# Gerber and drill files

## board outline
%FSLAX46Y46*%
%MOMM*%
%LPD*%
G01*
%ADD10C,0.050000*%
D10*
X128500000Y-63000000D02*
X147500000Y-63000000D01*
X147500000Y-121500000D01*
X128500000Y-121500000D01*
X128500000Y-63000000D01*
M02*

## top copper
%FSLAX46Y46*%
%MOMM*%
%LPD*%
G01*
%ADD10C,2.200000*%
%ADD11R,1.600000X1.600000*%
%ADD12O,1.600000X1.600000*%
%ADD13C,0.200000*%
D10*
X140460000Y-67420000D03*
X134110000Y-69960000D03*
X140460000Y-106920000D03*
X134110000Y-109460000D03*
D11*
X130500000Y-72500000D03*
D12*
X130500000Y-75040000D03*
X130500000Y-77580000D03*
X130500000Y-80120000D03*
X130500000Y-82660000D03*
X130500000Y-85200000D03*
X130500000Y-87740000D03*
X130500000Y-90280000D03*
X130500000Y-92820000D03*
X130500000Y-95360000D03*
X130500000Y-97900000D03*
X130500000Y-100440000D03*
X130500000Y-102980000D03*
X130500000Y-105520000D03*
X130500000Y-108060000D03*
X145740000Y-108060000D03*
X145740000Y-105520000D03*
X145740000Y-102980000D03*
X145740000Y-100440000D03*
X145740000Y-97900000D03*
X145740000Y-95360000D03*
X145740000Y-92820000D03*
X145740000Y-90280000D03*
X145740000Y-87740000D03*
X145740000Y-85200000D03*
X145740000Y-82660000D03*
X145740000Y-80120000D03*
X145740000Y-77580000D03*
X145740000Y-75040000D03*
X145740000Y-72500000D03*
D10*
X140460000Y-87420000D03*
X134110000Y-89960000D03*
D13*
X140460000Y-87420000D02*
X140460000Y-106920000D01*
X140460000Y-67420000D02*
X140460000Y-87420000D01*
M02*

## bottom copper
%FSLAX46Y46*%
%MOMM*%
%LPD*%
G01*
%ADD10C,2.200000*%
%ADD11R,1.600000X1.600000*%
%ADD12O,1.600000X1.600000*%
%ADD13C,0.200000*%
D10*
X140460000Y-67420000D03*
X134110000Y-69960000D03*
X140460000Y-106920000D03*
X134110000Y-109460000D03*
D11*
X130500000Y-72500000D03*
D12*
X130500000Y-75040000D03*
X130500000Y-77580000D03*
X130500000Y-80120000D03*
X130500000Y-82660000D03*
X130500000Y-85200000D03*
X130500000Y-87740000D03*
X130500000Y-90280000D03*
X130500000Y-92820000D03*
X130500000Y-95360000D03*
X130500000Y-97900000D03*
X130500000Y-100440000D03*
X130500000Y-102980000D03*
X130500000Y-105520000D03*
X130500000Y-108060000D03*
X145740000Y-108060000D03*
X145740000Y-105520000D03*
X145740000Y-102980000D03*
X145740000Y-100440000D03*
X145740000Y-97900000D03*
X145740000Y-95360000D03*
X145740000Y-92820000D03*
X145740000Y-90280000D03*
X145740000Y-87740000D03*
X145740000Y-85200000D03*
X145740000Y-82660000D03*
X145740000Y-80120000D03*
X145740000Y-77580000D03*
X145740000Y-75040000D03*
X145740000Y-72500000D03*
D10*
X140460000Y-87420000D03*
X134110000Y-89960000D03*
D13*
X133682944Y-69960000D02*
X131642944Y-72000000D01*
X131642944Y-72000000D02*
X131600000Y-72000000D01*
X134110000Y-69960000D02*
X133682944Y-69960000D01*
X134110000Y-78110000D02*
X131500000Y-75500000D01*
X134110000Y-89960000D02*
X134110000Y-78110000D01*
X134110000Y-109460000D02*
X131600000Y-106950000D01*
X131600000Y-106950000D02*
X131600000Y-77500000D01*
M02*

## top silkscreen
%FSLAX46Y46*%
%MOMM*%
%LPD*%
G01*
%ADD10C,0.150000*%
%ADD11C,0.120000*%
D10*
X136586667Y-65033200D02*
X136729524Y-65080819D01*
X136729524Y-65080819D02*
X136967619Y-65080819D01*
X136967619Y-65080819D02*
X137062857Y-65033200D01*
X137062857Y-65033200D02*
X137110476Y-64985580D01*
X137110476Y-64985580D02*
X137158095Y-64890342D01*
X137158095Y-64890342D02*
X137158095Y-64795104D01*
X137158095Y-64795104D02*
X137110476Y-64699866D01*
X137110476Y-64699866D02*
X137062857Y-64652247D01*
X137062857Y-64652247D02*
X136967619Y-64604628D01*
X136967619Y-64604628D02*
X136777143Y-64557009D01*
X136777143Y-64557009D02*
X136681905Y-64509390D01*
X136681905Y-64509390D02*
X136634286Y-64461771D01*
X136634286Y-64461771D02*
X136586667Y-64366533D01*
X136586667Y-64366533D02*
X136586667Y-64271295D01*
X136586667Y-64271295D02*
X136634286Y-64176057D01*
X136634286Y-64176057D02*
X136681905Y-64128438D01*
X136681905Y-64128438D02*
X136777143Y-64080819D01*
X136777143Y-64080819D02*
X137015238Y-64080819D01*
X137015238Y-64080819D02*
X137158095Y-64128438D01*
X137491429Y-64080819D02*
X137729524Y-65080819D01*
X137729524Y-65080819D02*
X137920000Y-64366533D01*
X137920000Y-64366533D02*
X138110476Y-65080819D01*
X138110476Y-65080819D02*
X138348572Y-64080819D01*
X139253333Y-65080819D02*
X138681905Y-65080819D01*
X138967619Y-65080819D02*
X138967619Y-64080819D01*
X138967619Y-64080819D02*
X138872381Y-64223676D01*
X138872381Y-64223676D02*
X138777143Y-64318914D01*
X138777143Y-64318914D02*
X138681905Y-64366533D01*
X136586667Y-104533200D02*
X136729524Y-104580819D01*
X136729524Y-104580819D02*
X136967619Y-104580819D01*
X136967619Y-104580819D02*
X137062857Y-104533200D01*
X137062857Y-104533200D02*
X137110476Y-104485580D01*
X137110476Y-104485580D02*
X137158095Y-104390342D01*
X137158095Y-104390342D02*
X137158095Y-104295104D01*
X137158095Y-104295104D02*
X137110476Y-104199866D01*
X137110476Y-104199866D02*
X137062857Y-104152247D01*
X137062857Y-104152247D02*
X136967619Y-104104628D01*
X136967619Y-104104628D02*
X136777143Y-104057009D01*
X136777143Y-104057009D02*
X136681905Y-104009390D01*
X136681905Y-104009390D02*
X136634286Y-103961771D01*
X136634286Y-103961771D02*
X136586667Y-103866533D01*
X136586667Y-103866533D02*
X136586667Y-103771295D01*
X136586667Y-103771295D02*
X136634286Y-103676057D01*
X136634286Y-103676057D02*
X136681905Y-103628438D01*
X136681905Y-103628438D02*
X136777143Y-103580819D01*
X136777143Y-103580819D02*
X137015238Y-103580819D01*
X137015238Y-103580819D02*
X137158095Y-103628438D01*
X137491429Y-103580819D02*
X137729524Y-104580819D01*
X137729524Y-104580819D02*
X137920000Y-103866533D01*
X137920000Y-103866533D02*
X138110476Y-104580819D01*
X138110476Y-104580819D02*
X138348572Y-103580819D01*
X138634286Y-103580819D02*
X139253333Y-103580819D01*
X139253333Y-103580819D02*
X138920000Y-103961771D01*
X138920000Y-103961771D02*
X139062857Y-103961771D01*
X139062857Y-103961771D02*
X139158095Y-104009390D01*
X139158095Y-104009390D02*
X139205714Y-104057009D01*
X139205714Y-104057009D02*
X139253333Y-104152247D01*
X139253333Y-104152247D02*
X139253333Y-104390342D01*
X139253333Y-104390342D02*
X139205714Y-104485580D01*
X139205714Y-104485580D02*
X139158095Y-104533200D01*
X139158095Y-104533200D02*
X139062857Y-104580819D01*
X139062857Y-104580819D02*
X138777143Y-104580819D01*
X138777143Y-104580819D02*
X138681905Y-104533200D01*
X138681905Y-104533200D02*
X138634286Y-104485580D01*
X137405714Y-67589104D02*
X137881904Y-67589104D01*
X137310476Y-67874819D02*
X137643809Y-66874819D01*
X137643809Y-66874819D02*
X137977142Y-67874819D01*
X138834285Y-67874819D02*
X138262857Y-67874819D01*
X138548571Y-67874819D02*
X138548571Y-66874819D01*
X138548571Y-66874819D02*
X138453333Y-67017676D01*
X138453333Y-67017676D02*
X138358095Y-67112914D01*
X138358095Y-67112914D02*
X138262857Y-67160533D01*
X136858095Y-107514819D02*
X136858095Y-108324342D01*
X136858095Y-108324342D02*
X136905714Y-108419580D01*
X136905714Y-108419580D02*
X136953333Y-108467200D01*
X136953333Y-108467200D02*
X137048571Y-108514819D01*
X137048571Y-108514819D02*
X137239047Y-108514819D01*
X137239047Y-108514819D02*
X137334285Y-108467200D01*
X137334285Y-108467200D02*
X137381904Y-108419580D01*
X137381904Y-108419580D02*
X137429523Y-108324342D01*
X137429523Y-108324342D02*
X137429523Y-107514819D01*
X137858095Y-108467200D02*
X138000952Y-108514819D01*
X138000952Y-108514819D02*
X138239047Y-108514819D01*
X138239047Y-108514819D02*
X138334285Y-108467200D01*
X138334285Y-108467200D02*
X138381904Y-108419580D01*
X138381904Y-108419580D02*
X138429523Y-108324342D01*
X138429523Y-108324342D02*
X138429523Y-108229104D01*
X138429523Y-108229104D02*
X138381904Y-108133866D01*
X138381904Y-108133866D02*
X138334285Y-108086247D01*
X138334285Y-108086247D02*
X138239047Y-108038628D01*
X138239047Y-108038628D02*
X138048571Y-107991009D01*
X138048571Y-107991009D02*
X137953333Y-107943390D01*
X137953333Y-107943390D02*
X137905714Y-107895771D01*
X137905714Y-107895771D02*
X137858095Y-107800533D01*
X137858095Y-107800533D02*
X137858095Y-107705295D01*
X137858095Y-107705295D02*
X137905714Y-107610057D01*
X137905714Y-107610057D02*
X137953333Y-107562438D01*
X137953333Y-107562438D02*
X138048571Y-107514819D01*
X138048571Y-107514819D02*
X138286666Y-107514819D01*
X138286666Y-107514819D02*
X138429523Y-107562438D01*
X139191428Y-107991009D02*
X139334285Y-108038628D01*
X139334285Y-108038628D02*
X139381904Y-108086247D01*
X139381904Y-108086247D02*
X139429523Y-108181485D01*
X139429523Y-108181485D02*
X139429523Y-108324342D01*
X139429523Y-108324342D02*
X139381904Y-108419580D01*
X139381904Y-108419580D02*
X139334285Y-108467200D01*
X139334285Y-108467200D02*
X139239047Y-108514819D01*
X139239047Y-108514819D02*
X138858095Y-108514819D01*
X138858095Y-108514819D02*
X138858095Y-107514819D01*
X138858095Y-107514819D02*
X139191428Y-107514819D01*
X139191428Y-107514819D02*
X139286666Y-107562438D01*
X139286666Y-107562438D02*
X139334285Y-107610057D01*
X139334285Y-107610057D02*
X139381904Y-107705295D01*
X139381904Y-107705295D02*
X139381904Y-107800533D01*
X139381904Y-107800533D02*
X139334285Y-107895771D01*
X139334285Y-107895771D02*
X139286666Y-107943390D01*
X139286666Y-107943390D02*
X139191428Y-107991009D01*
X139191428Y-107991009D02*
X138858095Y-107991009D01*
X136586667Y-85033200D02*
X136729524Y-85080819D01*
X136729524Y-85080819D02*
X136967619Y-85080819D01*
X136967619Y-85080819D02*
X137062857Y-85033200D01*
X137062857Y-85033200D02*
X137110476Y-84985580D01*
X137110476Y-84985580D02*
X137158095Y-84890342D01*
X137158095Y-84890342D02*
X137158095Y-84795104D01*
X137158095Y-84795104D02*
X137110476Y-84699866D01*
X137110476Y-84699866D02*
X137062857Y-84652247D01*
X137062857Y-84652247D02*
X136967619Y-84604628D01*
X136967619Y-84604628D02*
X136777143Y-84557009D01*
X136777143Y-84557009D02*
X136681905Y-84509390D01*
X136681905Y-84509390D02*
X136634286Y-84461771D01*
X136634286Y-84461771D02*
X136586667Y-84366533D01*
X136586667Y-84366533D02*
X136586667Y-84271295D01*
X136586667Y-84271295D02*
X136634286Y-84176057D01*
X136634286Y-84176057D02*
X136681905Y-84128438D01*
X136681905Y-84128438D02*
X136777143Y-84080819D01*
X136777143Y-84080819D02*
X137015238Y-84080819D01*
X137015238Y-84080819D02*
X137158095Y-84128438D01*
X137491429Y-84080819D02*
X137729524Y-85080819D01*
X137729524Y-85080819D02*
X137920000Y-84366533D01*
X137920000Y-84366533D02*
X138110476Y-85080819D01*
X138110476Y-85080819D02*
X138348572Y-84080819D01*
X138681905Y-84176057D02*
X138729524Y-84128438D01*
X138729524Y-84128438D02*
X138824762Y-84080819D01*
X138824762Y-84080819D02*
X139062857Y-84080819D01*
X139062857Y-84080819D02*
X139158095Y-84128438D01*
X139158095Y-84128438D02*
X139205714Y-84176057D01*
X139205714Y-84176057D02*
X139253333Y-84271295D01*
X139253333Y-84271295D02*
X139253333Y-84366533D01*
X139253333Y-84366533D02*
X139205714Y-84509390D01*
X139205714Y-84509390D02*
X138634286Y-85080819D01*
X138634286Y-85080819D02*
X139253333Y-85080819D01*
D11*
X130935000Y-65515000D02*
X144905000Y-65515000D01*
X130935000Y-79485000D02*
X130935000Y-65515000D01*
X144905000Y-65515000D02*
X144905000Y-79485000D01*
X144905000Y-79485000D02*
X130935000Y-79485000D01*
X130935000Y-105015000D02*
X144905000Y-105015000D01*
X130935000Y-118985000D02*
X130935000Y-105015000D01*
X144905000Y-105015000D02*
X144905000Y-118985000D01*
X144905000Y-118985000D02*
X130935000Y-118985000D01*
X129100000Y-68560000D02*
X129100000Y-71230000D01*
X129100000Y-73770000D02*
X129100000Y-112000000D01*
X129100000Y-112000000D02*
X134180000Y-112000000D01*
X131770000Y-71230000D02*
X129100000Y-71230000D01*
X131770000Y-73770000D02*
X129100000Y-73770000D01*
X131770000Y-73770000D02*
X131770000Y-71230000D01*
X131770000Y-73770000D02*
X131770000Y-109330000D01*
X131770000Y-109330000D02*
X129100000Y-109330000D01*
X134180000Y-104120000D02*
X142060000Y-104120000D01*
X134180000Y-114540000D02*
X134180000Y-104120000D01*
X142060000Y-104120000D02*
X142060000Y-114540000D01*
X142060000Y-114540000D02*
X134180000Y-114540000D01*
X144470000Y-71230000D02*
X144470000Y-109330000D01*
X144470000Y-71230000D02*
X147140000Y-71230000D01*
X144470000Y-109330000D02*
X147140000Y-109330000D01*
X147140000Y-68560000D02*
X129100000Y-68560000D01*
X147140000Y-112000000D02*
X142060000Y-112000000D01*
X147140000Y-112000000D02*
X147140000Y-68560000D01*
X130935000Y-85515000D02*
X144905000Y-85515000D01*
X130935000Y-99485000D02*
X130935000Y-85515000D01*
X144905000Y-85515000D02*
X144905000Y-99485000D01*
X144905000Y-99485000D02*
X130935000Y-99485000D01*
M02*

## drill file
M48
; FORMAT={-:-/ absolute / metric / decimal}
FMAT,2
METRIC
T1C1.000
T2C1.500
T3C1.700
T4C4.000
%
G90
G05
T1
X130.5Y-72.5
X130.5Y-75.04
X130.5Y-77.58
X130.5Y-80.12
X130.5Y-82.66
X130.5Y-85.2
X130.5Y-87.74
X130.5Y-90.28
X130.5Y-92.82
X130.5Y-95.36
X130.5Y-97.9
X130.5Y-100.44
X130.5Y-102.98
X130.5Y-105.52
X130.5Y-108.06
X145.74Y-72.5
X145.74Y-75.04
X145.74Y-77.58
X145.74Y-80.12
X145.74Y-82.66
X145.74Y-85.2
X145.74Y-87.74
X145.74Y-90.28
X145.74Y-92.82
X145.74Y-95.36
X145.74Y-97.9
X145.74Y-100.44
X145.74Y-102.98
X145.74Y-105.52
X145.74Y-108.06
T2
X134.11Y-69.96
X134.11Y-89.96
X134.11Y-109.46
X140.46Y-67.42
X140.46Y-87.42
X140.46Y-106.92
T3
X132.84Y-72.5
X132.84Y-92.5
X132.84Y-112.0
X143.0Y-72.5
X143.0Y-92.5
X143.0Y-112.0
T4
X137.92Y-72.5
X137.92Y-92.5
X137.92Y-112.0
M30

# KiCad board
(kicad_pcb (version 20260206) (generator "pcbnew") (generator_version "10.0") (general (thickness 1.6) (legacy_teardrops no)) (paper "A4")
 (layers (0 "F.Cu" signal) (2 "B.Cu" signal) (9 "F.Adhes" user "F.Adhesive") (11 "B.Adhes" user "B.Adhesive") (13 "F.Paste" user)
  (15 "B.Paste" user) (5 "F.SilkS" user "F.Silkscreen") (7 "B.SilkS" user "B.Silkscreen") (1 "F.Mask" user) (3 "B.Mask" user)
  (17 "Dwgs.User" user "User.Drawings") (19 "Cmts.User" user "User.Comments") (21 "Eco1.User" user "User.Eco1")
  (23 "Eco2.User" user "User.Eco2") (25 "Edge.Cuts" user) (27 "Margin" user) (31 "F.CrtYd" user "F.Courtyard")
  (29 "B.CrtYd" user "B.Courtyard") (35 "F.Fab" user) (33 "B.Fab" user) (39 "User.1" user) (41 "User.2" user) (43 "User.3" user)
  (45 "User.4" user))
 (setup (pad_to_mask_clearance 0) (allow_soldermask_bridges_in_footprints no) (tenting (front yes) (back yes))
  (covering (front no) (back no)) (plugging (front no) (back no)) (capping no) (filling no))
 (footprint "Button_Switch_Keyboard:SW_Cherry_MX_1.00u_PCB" (layer "F.Cu") (at 140.46 67.42)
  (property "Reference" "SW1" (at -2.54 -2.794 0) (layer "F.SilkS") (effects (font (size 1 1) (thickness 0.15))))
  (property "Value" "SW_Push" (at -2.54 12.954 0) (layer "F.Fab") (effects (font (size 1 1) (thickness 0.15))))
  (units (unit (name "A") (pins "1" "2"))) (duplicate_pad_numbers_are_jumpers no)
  (fp_line (start -9.525 -1.905) (end 4.445 -1.905) (stroke (width 0.12) (type solid)) (layer "F.SilkS"))
  (fp_line (start -9.525 12.065) (end -9.525 -1.905) (stroke (width 0.12) (type solid)) (layer "F.SilkS"))
  (fp_line (start 4.445 -1.905) (end 4.445 12.065) (stroke (width 0.12) (type solid)) (layer "F.SilkS"))
  (fp_line (start 4.445 12.065) (end -9.525 12.065) (stroke (width 0.12) (type solid)) (layer "F.SilkS"))
  (pad "" np_thru_hole circle (at -7.62 5.08) (size 1.7 1.7) (drill 1.7) (layers "*.Cu" "*.Mask"))
  (pad "" np_thru_hole circle (at -2.54 5.08) (size 4 4) (drill 4) (layers "*.Cu" "*.Mask"))
  (pad "" np_thru_hole circle (at 2.54 5.08) (size 1.7 1.7) (drill 1.7) (layers "*.Cu" "*.Mask"))
  (pad "1" thru_hole circle (at 0 0) (size 2.2 2.2) (drill 1.5) (layers "*.Cu" "*.Mask") (remove_unused_layers no) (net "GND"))
  (pad "2" thru_hole circle (at -6.35 2.54) (size 2.2 2.2) (drill 1.5) (layers "*.Cu" "*.Mask") (remove_unused_layers no)
   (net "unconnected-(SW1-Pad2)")))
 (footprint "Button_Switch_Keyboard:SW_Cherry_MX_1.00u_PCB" (layer "F.Cu") (at 140.46 106.92)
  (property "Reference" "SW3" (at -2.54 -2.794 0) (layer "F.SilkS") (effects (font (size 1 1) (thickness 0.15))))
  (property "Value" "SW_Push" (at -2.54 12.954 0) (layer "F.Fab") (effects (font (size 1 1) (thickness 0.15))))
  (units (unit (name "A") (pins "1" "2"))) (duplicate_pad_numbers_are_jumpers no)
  (fp_line (start -9.525 -1.905) (end 4.445 -1.905) (stroke (width 0.12) (type solid)) (layer "F.SilkS"))
  (fp_line (start -9.525 12.065) (end -9.525 -1.905) (stroke (width 0.12) (type solid)) (layer "F.SilkS"))
  (fp_line (start 4.445 -1.905) (end 4.445 12.065) (stroke (width 0.12) (type solid)) (layer "F.SilkS"))
  (fp_line (start 4.445 12.065) (end -9.525 12.065) (stroke (width 0.12) (type solid)) (layer "F.SilkS"))
  (pad "" np_thru_hole circle (at -7.62 5.08) (size 1.7 1.7) (drill 1.7) (layers "*.Cu" "*.Mask"))
  (pad "" np_thru_hole circle (at -2.54 5.08) (size 4 4) (drill 4) (layers "*.Cu" "*.Mask"))
  (pad "" np_thru_hole circle (at 2.54 5.08) (size 1.7 1.7) (drill 1.7) (layers "*.Cu" "*.Mask"))
  (pad "1" thru_hole circle (at 0 0) (size 2.2 2.2) (drill 1.5) (layers "*.Cu" "*.Mask") (remove_unused_layers no) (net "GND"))
  (pad "2" thru_hole circle (at -6.35 2.54) (size 2.2 2.2) (drill 1.5) (layers "*.Cu" "*.Mask") (remove_unused_layers no)
   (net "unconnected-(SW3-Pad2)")))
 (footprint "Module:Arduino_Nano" (layer "F.Cu") (at 130.5 72.5)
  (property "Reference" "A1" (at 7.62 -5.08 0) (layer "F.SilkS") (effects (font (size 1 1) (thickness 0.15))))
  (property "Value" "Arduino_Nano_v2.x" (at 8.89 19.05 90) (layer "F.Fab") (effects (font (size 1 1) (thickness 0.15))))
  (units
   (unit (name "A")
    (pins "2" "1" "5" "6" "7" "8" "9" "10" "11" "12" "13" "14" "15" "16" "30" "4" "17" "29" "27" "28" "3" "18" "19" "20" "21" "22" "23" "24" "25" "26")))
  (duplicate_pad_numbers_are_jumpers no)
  (fp_line (start -1.4 -3.94) (end -1.4 -1.27) (stroke (width 0.12) (type solid)) (layer "F.SilkS"))
  (fp_line (start -1.4 1.27) (end -1.4 39.5) (stroke (width 0.12) (type solid)) (layer "F.SilkS"))
  (fp_line (start -1.4 39.5) (end 3.68 39.5) (stroke (width 0.12) (type solid)) (layer "F.SilkS"))
  (fp_line (start 1.27 -1.27) (end -1.4 -1.27) (stroke (width 0.12) (type solid)) (layer "F.SilkS"))
  (fp_line (start 1.27 1.27) (end -1.4 1.27) (stroke (width 0.12) (type solid)) (layer "F.SilkS"))
  (fp_line (start 1.27 1.27) (end 1.27 -1.27) (stroke (width 0.12) (type solid)) (layer "F.SilkS"))
  (fp_line (start 1.27 1.27) (end 1.27 36.83) (stroke (width 0.12) (type solid)) (layer "F.SilkS"))
  (fp_line (start 1.27 36.83) (end -1.4 36.83) (stroke (width 0.12) (type solid)) (layer "F.SilkS"))
  (fp_line (start 3.68 31.62) (end 11.56 31.62) (stroke (width 0.12) (type solid)) (layer "F.SilkS"))
  (fp_line (start 3.68 42.04) (end 3.68 31.62) (stroke (width 0.12) (type solid)) (layer "F.SilkS"))
  (fp_line (start 11.56 31.62) (end 11.56 42.04) (stroke (width 0.12) (type solid)) (layer "F.SilkS"))
  (fp_line (start 11.56 42.04) (end 3.68 42.04) (stroke (width 0.12) (type solid)) (layer "F.SilkS"))
  (fp_line (start 13.97 -1.27) (end 13.97 36.83) (stroke (width 0.12) (type solid)) (layer "F.SilkS"))
  (fp_line (start 13.97 -1.27) (end 16.64 -1.27) (stroke (width 0.12) (type solid)) (layer "F.SilkS"))
  (fp_line (start 13.97 36.83) (end 16.64 36.83) (stroke (width 0.12) (type solid)) (layer "F.SilkS"))
  (fp_line (start 16.64 -3.94) (end -1.4 -3.94) (stroke (width 0.12) (type solid)) (layer "F.SilkS"))
  (fp_line (start 16.64 39.5) (end 11.56 39.5) (stroke (width 0.12) (type solid)) (layer "F.SilkS"))
  (fp_line (start 16.64 39.5) (end 16.64 -3.94) (stroke (width 0.12) (type solid)) (layer "F.SilkS"))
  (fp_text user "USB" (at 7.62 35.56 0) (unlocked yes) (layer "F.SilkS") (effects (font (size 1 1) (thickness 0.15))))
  (pad "1" thru_hole rect (at 0 0) (size 1.6 1.6) (drill 1) (layers "*.Cu" "*.Mask") (remove_unused_layers no)
   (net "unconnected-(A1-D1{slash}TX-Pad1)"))
  (pad "2" thru_hole oval (at 0 2.54) (size 1.6 1.6) (drill 1) (layers "*.Cu" "*.Mask") (remove_unused_layers no)
   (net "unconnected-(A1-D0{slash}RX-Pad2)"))
  (pad "3" thru_hole oval (at 0 5.08) (size 1.6 1.6) (drill 1) (layers "*.Cu" "*.Mask") (remove_unused_layers no)
   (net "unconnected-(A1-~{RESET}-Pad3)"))
  (pad "4" thru_hole oval (at 0 7.62) (size 1.6 1.6) (drill 1) (layers "*.Cu" "*.Mask") (remove_unused_layers no) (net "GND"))
  (pad "5" thru_hole oval (at 0 10.16) (size 1.6 1.6) (drill 1) (layers "*.Cu" "*.Mask") (remove_unused_layers no)
   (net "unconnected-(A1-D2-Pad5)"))
  (pad "6" thru_hole oval (at 0 12.7) (size 1.6 1.6) (drill 1) (layers "*.Cu" "*.Mask") (remove_unused_layers no)
   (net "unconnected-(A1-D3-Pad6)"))
  (pad "7" thru_hole oval (at 0 15.24) (size 1.6 1.6) (drill 1) (layers "*.Cu" "*.Mask") (remove_unused_layers no)
   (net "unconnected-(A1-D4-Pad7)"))
  (pad "8" thru_hole oval (at 0 17.78) (size 1.6 1.6) (drill 1) (layers "*.Cu" "*.Mask") (remove_unused_layers no)
   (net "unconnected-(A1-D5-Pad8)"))
  (pad "9" thru_hole oval (at 0 20.32) (size 1.6 1.6) (drill 1) (layers "*.Cu" "*.Mask") (remove_unused_layers no) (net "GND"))
  (pad "10" thru_hole oval (at 0 22.86) (size 1.6 1.6) (drill 1) (layers "*.Cu" "*.Mask") (remove_unused_layers no) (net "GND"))
  (pad "11" thru_hole oval (at 0 25.4) (size 1.6 1.6) (drill 1) (layers "*.Cu" "*.Mask") (remove_unused_layers no) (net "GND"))
  (pad "12" thru_hole oval (at 0 27.94) (size 1.6 1.6) (drill 1) (layers "*.Cu" "*.Mask") (remove_unused_layers no)
   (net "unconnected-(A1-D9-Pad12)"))
  (pad "13" thru_hole oval (at 0 30.48) (size 1.6 1.6) (drill 1) (layers "*.Cu" "*.Mask") (remove_unused_layers no)
   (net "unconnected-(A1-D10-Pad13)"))
  (pad "14" thru_hole oval (at 0 33.02) (size 1.6 1.6) (drill 1) (layers "*.Cu" "*.Mask") (remove_unused_layers no)
   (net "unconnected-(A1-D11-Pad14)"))
  (pad "15" thru_hole oval (at 0 35.56) (size 1.6 1.6) (drill 1) (layers "*.Cu" "*.Mask") (remove_unused_layers no)
   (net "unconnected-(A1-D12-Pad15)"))
  (pad "16" thru_hole oval (at 15.24 35.56) (size 1.6 1.6) (drill 1) (layers "*.Cu" "*.Mask") (remove_unused_layers no)
   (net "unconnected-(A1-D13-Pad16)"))
  (pad "17" thru_hole oval (at 15.24 33.02) (size 1.6 1.6) (drill 1) (layers "*.Cu" "*.Mask") (remove_unused_layers no)
   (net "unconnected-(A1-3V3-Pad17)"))
  (pad "18" thru_hole oval (at 15.24 30.48) (size 1.6 1.6) (drill 1) (layers "*.Cu" "*.Mask") (remove_unused_layers no)
   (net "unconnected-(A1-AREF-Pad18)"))
  (pad "19" thru_hole oval (at 15.24 27.94) (size 1.6 1.6) (drill 1) (layers "*.Cu" "*.Mask") (remove_unused_layers no)
   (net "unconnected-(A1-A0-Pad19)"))
  (pad "20" thru_hole oval (at 15.24 25.4) (size 1.6 1.6) (drill 1) (layers "*.Cu" "*.Mask") (remove_unused_layers no)
   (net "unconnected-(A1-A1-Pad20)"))
  (pad "21" thru_hole oval (at 15.24 22.86) (size 1.6 1.6) (drill 1) (layers "*.Cu" "*.Mask") (remove_unused_layers no)
   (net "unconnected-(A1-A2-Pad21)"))
  (pad "22" thru_hole oval (at 15.24 20.32) (size 1.6 1.6) (drill 1) (layers "*.Cu" "*.Mask") (remove_unused_layers no)
   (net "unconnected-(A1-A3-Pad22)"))
  (pad "23" thru_hole oval (at 15.24 17.78) (size 1.6 1.6) (drill 1) (layers "*.Cu" "*.Mask") (remove_unused_layers no)
   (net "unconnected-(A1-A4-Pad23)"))
  (pad "24" thru_hole oval (at 15.24 15.24) (size 1.6 1.6) (drill 1) (layers "*.Cu" "*.Mask") (remove_unused_layers no)
   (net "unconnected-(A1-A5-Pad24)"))
  (pad "25" thru_hole oval (at 15.24 12.7) (size 1.6 1.6) (drill 1) (layers "*.Cu" "*.Mask") (remove_unused_layers no)
   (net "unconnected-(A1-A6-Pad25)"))
  (pad "26" thru_hole oval (at 15.24 10.16) (size 1.6 1.6) (drill 1) (layers "*.Cu" "*.Mask") (remove_unused_layers no)
   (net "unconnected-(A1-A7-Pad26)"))
  (pad "27" thru_hole oval (at 15.24 7.62) (size 1.6 1.6) (drill 1) (layers "*.Cu" "*.Mask") (remove_unused_layers no)
   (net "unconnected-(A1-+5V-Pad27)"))
  (pad "28" thru_hole oval (at 15.24 5.08) (size 1.6 1.6) (drill 1) (layers "*.Cu" "*.Mask") (remove_unused_layers no)
   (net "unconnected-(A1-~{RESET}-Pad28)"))
  (pad "29" thru_hole oval (at 15.24 2.54) (size 1.6 1.6) (drill 1) (layers "*.Cu" "*.Mask") (remove_unused_layers no)
   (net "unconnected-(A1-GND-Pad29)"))
  (pad "30" thru_hole oval (at 15.24 0) (size 1.6 1.6) (drill 1) (layers "*.Cu" "*.Mask") (remove_unused_layers no)
   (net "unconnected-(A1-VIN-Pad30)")))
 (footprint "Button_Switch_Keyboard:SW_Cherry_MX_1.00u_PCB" (layer "F.Cu") (at 140.46 87.42)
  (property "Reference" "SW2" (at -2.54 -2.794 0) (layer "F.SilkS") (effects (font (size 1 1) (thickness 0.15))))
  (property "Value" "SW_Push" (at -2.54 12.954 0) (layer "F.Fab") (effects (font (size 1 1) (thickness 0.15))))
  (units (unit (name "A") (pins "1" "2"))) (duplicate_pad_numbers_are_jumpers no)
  (fp_line (start -9.525 -1.905) (end 4.445 -1.905) (stroke (width 0.12) (type solid)) (layer "F.SilkS"))
  (fp_line (start -9.525 12.065) (end -9.525 -1.905) (stroke (width 0.12) (type solid)) (layer "F.SilkS"))
  (fp_line (start 4.445 -1.905) (end 4.445 12.065) (stroke (width 0.12) (type solid)) (layer "F.SilkS"))
  (fp_line (start 4.445 12.065) (end -9.525 12.065) (stroke (width 0.12) (type solid)) (layer "F.SilkS"))
  (pad "" np_thru_hole circle (at -7.62 5.08) (size 1.7 1.7) (drill 1.7) (layers "*.Cu" "*.Mask"))
  (pad "" np_thru_hole circle (at -2.54 5.08) (size 4 4) (drill 4) (layers "*.Cu" "*.Mask"))
  (pad "" np_thru_hole circle (at 2.54 5.08) (size 1.7 1.7) (drill 1.7) (layers "*.Cu" "*.Mask"))
  (pad "1" thru_hole circle (at 0 0) (size 2.2 2.2) (drill 1.5) (layers "*.Cu" "*.Mask") (remove_unused_layers no) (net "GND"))
  (pad "2" thru_hole circle (at -6.35 2.54) (size 2.2 2.2) (drill 1.5) (layers "*.Cu" "*.Mask") (remove_unused_layers no)
   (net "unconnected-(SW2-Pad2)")))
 (gr_rect (start 128.5 63) (end 147.5 121.5) (stroke (width 0.05) (type default)) (fill no) (locked yes) (layer "Edge.Cuts"))
 (segment (start 140.46 87.42) (end 140.46 106.92) (width 0.2) (layer "F.Cu") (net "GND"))
 (segment (start 140.46 67.42) (end 140.46 87.42) (width 0.2) (layer "F.Cu") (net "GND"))
 (segment (start 133.682944 69.96) (end 131.642944 72) (width 0.2) (layer "B.Cu") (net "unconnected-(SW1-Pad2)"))
 (segment (start 131.642944 72) (end 131.6 72) (width 0.2) (layer "B.Cu") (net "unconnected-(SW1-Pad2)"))
 (segment (start 134.11 69.96) (end 133.682944 69.96) (width 0.2) (layer "B.Cu") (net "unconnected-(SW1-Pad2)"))
 (segment (start 134.11 78.11) (end 131.5 75.5) (width 0.2) (layer "B.Cu") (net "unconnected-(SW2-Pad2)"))
 (segment (start 134.11 89.96) (end 134.11 78.11) (width 0.2) (layer "B.Cu") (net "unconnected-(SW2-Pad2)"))
 (segment (start 134.11 109.46) (end 131.6 106.95) (width 0.2) (layer "B.Cu") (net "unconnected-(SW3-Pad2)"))
 (segment (start 131.6 106.95) (end 131.6 77.5) (width 0.2) (layer "B.Cu") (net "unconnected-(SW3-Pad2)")))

